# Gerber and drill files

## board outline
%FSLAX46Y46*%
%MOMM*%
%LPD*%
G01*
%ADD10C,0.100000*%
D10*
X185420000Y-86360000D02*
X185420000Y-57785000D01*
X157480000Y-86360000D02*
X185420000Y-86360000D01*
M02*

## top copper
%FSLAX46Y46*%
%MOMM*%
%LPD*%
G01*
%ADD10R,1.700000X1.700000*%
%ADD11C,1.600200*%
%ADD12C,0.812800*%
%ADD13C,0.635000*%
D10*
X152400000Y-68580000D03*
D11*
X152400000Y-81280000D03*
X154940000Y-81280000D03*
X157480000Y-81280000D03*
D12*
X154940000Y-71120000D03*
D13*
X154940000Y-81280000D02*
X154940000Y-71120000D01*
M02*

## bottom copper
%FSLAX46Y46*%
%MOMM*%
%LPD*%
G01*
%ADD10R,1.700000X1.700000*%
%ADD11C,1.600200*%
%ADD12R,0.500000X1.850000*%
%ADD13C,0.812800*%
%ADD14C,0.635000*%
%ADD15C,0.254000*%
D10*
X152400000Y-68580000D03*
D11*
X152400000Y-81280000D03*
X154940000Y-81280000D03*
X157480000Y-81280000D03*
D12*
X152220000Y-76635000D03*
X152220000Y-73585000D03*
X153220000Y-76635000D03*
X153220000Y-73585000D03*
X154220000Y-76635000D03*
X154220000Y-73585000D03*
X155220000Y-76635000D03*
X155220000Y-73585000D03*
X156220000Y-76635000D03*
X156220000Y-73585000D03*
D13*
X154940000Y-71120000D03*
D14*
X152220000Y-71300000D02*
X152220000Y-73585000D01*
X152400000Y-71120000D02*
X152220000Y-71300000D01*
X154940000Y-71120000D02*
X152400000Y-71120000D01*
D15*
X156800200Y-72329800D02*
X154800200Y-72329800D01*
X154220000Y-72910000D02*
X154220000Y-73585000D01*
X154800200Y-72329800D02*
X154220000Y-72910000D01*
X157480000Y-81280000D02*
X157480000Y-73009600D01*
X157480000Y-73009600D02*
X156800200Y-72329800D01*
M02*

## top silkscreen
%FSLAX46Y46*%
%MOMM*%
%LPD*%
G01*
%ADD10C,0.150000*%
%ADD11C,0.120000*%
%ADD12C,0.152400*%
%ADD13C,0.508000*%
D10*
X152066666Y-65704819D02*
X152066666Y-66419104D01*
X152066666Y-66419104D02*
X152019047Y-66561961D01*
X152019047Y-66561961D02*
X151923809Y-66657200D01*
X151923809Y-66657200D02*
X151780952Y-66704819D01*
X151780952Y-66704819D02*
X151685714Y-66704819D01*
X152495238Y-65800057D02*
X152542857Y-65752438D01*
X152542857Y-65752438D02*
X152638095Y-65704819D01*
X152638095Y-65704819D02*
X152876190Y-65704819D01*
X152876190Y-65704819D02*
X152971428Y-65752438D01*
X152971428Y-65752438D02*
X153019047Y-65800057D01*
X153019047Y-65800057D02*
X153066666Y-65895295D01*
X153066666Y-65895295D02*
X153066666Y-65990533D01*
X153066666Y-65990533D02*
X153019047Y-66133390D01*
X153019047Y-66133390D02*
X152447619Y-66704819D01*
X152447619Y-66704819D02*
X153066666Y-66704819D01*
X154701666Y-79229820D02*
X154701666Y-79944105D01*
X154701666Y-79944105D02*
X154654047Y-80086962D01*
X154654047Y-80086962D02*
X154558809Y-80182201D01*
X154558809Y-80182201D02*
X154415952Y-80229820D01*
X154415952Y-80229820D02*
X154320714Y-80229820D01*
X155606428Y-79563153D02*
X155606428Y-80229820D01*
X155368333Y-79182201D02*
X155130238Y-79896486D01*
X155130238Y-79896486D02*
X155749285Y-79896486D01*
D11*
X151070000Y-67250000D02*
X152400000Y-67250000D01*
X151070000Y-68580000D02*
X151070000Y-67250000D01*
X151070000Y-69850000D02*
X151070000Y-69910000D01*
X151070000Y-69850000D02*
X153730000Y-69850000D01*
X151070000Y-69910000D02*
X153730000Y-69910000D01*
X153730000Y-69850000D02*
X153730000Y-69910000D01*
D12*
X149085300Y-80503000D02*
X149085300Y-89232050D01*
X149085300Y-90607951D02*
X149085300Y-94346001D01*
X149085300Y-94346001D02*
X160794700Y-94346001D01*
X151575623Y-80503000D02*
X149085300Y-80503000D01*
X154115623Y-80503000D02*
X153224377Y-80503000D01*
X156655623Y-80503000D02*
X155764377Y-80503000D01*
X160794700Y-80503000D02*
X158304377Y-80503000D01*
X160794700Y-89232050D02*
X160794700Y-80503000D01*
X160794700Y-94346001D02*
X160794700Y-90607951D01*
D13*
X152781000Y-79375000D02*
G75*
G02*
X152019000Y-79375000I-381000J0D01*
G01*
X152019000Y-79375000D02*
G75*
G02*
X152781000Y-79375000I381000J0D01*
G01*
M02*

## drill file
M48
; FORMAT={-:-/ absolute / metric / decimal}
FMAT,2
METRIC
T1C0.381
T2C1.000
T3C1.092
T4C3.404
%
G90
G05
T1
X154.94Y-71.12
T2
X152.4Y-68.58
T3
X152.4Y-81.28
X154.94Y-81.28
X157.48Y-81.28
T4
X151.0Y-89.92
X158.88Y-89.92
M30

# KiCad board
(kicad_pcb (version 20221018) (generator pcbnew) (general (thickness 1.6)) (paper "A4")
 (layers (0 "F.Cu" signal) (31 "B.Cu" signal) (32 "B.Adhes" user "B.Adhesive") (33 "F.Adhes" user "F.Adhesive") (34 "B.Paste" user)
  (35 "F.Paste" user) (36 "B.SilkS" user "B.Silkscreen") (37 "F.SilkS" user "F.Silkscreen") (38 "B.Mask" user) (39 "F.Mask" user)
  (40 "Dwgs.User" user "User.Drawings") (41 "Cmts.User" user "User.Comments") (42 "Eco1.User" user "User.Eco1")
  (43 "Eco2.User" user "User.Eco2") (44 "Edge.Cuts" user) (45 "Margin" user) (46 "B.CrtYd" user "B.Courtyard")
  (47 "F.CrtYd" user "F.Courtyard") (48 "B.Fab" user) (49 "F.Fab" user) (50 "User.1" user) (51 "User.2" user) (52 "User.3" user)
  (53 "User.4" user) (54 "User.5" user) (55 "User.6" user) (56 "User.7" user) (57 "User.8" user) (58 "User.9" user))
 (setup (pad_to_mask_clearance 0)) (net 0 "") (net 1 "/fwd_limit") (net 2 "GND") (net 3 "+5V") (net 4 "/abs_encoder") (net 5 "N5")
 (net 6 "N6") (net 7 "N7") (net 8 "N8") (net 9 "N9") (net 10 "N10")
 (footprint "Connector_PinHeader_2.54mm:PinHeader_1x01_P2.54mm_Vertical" (layer "F.Cu") (at 152.4 68.58)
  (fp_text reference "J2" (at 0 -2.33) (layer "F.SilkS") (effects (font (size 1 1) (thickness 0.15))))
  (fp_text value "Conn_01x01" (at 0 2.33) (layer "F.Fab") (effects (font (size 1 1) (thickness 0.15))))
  (fp_line (start -1.33 -1.33) (end 0 -1.33) (stroke (width 0.12) (type solid)) (layer "F.SilkS"))
  (fp_line (start -1.33 0) (end -1.33 -1.33) (stroke (width 0.12) (type solid)) (layer "F.SilkS"))
  (fp_line (start -1.33 1.27) (end -1.33 1.33) (stroke (width 0.12) (type solid)) (layer "F.SilkS"))
  (fp_line (start -1.33 1.27) (end 1.33 1.27) (stroke (width 0.12) (type solid)) (layer "F.SilkS"))
  (fp_line (start -1.33 1.33) (end 1.33 1.33) (stroke (width 0.12) (type solid)) (layer "F.SilkS"))
  (fp_line (start 1.33 1.27) (end 1.33 1.33) (stroke (width 0.12) (type solid)) (layer "F.SilkS"))
  (pad "1" thru_hole rect (at 0 0) (size 1.7 1.7) (drill 1) (layers "*.Cu" "*.Mask") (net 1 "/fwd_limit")))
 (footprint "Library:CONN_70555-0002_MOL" (layer "F.Cu") (at 152.4 81.28)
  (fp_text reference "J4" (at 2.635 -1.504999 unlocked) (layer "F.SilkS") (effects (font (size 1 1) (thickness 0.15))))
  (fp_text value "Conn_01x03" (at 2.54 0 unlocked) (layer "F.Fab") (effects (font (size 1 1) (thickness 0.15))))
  (fp_line (start -3.3147 -0.777) (end -3.3147 7.95205) (stroke (width 0.1524) (type solid)) (layer "F.SilkS"))
  (fp_line (start -3.3147 9.327951) (end -3.3147 13.066001) (stroke (width 0.1524) (type solid)) (layer "F.SilkS"))
  (fp_line (start -3.3147 13.066001) (end 8.3947 13.066001) (stroke (width 0.1524) (type solid)) (layer "F.SilkS"))
  (fp_line (start -0.824377 -0.777) (end -3.3147 -0.777) (stroke (width 0.1524) (type solid)) (layer "F.SilkS"))
  (fp_line (start 1.715623 -0.777) (end 0.824377 -0.777) (stroke (width 0.1524) (type solid)) (layer "F.SilkS"))
  (fp_line (start 4.255623 -0.777) (end 3.364377 -0.777) (stroke (width 0.1524) (type solid)) (layer "F.SilkS"))
  (fp_line (start 8.3947 -0.777) (end 5.904377 -0.777) (stroke (width 0.1524) (type solid)) (layer "F.SilkS"))
  (fp_line (start 8.3947 7.95205) (end 8.3947 -0.777) (stroke (width 0.1524) (type solid)) (layer "F.SilkS"))
  (fp_line (start 8.3947 13.066001) (end 8.3947 9.327951) (stroke (width 0.1524) (type solid)) (layer "F.SilkS"))
  (fp_circle (center 0 -1.905) (end 0.381 -1.905) (stroke (width 0.508) (type solid)) (fill none) (layer "F.SilkS"))
  (pad "" np_thru_hole circle (at -1.4 8.640001) (size 3.4036 3.4036) (drill 3.4036) (layers "*.Cu" "*.Mask"))
  (pad "" np_thru_hole circle (at 6.48 8.640001) (size 3.4036 3.4036) (drill 3.4036) (layers "*.Cu" "*.Mask"))
  (pad "1" thru_hole circle (at 0 0) (size 1.6002 1.6002) (drill 1.0922) (layers "*.Cu" "*.Mask") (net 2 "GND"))
  (pad "2" thru_hole circle (at 2.54 0) (size 1.6002 1.6002) (drill 1.0922) (layers "*.Cu" "*.Mask") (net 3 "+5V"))
  (pad "3" thru_hole circle (at 5.08 0) (size 1.6002 1.6002) (drill 1.0922) (layers "*.Cu" "*.Mask") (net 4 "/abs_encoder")))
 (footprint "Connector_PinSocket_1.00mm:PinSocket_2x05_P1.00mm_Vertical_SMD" (layer "B.Cu") (at 154.22 75.11 -90)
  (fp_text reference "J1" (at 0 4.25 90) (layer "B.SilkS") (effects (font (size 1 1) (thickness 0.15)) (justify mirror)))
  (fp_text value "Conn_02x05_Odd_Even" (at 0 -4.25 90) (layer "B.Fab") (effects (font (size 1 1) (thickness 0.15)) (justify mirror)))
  (pad "1" smd rect (at 1.525 2 270) (size 1.85 0.5) (layers "B.Cu" "B.Paste" "B.Mask") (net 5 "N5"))
  (pad "2" smd rect (at -1.525 2 270) (size 1.85 0.5) (layers "B.Cu" "B.Paste" "B.Mask") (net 3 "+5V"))
  (pad "3" smd rect (at 1.525 1 270) (size 1.85 0.5) (layers "B.Cu" "B.Paste" "B.Mask") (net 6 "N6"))
  (pad "4" smd rect (at -1.525 1 270) (size 1.85 0.5) (layers "B.Cu" "B.Paste" "B.Mask") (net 1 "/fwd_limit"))
  (pad "5" smd rect (at 1.525 0 270) (size 1.85 0.5) (layers "B.Cu" "B.Paste" "B.Mask") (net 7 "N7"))
  (pad "6" smd rect (at -1.525 0 270) (size 1.85 0.5) (layers "B.Cu" "B.Paste" "B.Mask") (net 4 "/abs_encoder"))
  (pad "7" smd rect (at 1.525 -1 270) (size 1.85 0.5) (layers "B.Cu" "B.Paste" "B.Mask") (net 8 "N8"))
  (pad "8" smd rect (at -1.525 -1 270) (size 1.85 0.5) (layers "B.Cu" "B.Paste" "B.Mask") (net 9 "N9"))
  (pad "9" smd rect (at 1.525 -2 270) (size 1.85 0.5) (layers "B.Cu" "B.Paste" "B.Mask") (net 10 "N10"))
  (pad "10" smd rect (at -1.525 -2 270) (size 1.85 0.5) (layers "B.Cu" "B.Paste" "B.Mask") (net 2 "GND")))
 (gr_line (start 185.42 86.36) (end 185.42 57.785) (stroke (width 0.1) (type default)) (layer "Edge.Cuts"))
 (gr_line (start 157.48 86.36) (end 185.42 86.36) (stroke (width 0.1) (type default)) (layer "Edge.Cuts"))
 (segment (start 154.94 81.28) (end 154.94 71.12) (width 0.635) (layer "F.Cu") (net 3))
 (via (at 154.94 71.12) (size 0.8128) (drill 0.381) (layers "F.Cu" "B.Cu") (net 3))
 (segment (start 152.22 71.3) (end 152.22 73.585) (width 0.635) (layer "B.Cu") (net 3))
 (segment (start 152.4 71.12) (end 152.22 71.3) (width 0.635) (layer "B.Cu") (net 3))
 (segment (start 154.94 71.12) (end 152.4 71.12) (width 0.635) (layer "B.Cu") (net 3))
 (segment (start 156.8002 72.3298) (end 154.8002 72.3298) (width 0.254) (layer "B.Cu") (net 4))
 (segment (start 154.22 72.91) (end 154.22 73.585) (width 0.254) (layer "B.Cu") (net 4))
 (segment (start 154.8002 72.3298) (end 154.22 72.91) (width 0.254) (layer "B.Cu") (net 4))
 (segment (start 157.48 81.28) (end 157.48 73.0096) (width 0.254) (layer "B.Cu") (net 4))
 (segment (start 157.48 73.0096) (end 156.8002 72.3298) (width 0.254) (layer "B.Cu") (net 4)))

